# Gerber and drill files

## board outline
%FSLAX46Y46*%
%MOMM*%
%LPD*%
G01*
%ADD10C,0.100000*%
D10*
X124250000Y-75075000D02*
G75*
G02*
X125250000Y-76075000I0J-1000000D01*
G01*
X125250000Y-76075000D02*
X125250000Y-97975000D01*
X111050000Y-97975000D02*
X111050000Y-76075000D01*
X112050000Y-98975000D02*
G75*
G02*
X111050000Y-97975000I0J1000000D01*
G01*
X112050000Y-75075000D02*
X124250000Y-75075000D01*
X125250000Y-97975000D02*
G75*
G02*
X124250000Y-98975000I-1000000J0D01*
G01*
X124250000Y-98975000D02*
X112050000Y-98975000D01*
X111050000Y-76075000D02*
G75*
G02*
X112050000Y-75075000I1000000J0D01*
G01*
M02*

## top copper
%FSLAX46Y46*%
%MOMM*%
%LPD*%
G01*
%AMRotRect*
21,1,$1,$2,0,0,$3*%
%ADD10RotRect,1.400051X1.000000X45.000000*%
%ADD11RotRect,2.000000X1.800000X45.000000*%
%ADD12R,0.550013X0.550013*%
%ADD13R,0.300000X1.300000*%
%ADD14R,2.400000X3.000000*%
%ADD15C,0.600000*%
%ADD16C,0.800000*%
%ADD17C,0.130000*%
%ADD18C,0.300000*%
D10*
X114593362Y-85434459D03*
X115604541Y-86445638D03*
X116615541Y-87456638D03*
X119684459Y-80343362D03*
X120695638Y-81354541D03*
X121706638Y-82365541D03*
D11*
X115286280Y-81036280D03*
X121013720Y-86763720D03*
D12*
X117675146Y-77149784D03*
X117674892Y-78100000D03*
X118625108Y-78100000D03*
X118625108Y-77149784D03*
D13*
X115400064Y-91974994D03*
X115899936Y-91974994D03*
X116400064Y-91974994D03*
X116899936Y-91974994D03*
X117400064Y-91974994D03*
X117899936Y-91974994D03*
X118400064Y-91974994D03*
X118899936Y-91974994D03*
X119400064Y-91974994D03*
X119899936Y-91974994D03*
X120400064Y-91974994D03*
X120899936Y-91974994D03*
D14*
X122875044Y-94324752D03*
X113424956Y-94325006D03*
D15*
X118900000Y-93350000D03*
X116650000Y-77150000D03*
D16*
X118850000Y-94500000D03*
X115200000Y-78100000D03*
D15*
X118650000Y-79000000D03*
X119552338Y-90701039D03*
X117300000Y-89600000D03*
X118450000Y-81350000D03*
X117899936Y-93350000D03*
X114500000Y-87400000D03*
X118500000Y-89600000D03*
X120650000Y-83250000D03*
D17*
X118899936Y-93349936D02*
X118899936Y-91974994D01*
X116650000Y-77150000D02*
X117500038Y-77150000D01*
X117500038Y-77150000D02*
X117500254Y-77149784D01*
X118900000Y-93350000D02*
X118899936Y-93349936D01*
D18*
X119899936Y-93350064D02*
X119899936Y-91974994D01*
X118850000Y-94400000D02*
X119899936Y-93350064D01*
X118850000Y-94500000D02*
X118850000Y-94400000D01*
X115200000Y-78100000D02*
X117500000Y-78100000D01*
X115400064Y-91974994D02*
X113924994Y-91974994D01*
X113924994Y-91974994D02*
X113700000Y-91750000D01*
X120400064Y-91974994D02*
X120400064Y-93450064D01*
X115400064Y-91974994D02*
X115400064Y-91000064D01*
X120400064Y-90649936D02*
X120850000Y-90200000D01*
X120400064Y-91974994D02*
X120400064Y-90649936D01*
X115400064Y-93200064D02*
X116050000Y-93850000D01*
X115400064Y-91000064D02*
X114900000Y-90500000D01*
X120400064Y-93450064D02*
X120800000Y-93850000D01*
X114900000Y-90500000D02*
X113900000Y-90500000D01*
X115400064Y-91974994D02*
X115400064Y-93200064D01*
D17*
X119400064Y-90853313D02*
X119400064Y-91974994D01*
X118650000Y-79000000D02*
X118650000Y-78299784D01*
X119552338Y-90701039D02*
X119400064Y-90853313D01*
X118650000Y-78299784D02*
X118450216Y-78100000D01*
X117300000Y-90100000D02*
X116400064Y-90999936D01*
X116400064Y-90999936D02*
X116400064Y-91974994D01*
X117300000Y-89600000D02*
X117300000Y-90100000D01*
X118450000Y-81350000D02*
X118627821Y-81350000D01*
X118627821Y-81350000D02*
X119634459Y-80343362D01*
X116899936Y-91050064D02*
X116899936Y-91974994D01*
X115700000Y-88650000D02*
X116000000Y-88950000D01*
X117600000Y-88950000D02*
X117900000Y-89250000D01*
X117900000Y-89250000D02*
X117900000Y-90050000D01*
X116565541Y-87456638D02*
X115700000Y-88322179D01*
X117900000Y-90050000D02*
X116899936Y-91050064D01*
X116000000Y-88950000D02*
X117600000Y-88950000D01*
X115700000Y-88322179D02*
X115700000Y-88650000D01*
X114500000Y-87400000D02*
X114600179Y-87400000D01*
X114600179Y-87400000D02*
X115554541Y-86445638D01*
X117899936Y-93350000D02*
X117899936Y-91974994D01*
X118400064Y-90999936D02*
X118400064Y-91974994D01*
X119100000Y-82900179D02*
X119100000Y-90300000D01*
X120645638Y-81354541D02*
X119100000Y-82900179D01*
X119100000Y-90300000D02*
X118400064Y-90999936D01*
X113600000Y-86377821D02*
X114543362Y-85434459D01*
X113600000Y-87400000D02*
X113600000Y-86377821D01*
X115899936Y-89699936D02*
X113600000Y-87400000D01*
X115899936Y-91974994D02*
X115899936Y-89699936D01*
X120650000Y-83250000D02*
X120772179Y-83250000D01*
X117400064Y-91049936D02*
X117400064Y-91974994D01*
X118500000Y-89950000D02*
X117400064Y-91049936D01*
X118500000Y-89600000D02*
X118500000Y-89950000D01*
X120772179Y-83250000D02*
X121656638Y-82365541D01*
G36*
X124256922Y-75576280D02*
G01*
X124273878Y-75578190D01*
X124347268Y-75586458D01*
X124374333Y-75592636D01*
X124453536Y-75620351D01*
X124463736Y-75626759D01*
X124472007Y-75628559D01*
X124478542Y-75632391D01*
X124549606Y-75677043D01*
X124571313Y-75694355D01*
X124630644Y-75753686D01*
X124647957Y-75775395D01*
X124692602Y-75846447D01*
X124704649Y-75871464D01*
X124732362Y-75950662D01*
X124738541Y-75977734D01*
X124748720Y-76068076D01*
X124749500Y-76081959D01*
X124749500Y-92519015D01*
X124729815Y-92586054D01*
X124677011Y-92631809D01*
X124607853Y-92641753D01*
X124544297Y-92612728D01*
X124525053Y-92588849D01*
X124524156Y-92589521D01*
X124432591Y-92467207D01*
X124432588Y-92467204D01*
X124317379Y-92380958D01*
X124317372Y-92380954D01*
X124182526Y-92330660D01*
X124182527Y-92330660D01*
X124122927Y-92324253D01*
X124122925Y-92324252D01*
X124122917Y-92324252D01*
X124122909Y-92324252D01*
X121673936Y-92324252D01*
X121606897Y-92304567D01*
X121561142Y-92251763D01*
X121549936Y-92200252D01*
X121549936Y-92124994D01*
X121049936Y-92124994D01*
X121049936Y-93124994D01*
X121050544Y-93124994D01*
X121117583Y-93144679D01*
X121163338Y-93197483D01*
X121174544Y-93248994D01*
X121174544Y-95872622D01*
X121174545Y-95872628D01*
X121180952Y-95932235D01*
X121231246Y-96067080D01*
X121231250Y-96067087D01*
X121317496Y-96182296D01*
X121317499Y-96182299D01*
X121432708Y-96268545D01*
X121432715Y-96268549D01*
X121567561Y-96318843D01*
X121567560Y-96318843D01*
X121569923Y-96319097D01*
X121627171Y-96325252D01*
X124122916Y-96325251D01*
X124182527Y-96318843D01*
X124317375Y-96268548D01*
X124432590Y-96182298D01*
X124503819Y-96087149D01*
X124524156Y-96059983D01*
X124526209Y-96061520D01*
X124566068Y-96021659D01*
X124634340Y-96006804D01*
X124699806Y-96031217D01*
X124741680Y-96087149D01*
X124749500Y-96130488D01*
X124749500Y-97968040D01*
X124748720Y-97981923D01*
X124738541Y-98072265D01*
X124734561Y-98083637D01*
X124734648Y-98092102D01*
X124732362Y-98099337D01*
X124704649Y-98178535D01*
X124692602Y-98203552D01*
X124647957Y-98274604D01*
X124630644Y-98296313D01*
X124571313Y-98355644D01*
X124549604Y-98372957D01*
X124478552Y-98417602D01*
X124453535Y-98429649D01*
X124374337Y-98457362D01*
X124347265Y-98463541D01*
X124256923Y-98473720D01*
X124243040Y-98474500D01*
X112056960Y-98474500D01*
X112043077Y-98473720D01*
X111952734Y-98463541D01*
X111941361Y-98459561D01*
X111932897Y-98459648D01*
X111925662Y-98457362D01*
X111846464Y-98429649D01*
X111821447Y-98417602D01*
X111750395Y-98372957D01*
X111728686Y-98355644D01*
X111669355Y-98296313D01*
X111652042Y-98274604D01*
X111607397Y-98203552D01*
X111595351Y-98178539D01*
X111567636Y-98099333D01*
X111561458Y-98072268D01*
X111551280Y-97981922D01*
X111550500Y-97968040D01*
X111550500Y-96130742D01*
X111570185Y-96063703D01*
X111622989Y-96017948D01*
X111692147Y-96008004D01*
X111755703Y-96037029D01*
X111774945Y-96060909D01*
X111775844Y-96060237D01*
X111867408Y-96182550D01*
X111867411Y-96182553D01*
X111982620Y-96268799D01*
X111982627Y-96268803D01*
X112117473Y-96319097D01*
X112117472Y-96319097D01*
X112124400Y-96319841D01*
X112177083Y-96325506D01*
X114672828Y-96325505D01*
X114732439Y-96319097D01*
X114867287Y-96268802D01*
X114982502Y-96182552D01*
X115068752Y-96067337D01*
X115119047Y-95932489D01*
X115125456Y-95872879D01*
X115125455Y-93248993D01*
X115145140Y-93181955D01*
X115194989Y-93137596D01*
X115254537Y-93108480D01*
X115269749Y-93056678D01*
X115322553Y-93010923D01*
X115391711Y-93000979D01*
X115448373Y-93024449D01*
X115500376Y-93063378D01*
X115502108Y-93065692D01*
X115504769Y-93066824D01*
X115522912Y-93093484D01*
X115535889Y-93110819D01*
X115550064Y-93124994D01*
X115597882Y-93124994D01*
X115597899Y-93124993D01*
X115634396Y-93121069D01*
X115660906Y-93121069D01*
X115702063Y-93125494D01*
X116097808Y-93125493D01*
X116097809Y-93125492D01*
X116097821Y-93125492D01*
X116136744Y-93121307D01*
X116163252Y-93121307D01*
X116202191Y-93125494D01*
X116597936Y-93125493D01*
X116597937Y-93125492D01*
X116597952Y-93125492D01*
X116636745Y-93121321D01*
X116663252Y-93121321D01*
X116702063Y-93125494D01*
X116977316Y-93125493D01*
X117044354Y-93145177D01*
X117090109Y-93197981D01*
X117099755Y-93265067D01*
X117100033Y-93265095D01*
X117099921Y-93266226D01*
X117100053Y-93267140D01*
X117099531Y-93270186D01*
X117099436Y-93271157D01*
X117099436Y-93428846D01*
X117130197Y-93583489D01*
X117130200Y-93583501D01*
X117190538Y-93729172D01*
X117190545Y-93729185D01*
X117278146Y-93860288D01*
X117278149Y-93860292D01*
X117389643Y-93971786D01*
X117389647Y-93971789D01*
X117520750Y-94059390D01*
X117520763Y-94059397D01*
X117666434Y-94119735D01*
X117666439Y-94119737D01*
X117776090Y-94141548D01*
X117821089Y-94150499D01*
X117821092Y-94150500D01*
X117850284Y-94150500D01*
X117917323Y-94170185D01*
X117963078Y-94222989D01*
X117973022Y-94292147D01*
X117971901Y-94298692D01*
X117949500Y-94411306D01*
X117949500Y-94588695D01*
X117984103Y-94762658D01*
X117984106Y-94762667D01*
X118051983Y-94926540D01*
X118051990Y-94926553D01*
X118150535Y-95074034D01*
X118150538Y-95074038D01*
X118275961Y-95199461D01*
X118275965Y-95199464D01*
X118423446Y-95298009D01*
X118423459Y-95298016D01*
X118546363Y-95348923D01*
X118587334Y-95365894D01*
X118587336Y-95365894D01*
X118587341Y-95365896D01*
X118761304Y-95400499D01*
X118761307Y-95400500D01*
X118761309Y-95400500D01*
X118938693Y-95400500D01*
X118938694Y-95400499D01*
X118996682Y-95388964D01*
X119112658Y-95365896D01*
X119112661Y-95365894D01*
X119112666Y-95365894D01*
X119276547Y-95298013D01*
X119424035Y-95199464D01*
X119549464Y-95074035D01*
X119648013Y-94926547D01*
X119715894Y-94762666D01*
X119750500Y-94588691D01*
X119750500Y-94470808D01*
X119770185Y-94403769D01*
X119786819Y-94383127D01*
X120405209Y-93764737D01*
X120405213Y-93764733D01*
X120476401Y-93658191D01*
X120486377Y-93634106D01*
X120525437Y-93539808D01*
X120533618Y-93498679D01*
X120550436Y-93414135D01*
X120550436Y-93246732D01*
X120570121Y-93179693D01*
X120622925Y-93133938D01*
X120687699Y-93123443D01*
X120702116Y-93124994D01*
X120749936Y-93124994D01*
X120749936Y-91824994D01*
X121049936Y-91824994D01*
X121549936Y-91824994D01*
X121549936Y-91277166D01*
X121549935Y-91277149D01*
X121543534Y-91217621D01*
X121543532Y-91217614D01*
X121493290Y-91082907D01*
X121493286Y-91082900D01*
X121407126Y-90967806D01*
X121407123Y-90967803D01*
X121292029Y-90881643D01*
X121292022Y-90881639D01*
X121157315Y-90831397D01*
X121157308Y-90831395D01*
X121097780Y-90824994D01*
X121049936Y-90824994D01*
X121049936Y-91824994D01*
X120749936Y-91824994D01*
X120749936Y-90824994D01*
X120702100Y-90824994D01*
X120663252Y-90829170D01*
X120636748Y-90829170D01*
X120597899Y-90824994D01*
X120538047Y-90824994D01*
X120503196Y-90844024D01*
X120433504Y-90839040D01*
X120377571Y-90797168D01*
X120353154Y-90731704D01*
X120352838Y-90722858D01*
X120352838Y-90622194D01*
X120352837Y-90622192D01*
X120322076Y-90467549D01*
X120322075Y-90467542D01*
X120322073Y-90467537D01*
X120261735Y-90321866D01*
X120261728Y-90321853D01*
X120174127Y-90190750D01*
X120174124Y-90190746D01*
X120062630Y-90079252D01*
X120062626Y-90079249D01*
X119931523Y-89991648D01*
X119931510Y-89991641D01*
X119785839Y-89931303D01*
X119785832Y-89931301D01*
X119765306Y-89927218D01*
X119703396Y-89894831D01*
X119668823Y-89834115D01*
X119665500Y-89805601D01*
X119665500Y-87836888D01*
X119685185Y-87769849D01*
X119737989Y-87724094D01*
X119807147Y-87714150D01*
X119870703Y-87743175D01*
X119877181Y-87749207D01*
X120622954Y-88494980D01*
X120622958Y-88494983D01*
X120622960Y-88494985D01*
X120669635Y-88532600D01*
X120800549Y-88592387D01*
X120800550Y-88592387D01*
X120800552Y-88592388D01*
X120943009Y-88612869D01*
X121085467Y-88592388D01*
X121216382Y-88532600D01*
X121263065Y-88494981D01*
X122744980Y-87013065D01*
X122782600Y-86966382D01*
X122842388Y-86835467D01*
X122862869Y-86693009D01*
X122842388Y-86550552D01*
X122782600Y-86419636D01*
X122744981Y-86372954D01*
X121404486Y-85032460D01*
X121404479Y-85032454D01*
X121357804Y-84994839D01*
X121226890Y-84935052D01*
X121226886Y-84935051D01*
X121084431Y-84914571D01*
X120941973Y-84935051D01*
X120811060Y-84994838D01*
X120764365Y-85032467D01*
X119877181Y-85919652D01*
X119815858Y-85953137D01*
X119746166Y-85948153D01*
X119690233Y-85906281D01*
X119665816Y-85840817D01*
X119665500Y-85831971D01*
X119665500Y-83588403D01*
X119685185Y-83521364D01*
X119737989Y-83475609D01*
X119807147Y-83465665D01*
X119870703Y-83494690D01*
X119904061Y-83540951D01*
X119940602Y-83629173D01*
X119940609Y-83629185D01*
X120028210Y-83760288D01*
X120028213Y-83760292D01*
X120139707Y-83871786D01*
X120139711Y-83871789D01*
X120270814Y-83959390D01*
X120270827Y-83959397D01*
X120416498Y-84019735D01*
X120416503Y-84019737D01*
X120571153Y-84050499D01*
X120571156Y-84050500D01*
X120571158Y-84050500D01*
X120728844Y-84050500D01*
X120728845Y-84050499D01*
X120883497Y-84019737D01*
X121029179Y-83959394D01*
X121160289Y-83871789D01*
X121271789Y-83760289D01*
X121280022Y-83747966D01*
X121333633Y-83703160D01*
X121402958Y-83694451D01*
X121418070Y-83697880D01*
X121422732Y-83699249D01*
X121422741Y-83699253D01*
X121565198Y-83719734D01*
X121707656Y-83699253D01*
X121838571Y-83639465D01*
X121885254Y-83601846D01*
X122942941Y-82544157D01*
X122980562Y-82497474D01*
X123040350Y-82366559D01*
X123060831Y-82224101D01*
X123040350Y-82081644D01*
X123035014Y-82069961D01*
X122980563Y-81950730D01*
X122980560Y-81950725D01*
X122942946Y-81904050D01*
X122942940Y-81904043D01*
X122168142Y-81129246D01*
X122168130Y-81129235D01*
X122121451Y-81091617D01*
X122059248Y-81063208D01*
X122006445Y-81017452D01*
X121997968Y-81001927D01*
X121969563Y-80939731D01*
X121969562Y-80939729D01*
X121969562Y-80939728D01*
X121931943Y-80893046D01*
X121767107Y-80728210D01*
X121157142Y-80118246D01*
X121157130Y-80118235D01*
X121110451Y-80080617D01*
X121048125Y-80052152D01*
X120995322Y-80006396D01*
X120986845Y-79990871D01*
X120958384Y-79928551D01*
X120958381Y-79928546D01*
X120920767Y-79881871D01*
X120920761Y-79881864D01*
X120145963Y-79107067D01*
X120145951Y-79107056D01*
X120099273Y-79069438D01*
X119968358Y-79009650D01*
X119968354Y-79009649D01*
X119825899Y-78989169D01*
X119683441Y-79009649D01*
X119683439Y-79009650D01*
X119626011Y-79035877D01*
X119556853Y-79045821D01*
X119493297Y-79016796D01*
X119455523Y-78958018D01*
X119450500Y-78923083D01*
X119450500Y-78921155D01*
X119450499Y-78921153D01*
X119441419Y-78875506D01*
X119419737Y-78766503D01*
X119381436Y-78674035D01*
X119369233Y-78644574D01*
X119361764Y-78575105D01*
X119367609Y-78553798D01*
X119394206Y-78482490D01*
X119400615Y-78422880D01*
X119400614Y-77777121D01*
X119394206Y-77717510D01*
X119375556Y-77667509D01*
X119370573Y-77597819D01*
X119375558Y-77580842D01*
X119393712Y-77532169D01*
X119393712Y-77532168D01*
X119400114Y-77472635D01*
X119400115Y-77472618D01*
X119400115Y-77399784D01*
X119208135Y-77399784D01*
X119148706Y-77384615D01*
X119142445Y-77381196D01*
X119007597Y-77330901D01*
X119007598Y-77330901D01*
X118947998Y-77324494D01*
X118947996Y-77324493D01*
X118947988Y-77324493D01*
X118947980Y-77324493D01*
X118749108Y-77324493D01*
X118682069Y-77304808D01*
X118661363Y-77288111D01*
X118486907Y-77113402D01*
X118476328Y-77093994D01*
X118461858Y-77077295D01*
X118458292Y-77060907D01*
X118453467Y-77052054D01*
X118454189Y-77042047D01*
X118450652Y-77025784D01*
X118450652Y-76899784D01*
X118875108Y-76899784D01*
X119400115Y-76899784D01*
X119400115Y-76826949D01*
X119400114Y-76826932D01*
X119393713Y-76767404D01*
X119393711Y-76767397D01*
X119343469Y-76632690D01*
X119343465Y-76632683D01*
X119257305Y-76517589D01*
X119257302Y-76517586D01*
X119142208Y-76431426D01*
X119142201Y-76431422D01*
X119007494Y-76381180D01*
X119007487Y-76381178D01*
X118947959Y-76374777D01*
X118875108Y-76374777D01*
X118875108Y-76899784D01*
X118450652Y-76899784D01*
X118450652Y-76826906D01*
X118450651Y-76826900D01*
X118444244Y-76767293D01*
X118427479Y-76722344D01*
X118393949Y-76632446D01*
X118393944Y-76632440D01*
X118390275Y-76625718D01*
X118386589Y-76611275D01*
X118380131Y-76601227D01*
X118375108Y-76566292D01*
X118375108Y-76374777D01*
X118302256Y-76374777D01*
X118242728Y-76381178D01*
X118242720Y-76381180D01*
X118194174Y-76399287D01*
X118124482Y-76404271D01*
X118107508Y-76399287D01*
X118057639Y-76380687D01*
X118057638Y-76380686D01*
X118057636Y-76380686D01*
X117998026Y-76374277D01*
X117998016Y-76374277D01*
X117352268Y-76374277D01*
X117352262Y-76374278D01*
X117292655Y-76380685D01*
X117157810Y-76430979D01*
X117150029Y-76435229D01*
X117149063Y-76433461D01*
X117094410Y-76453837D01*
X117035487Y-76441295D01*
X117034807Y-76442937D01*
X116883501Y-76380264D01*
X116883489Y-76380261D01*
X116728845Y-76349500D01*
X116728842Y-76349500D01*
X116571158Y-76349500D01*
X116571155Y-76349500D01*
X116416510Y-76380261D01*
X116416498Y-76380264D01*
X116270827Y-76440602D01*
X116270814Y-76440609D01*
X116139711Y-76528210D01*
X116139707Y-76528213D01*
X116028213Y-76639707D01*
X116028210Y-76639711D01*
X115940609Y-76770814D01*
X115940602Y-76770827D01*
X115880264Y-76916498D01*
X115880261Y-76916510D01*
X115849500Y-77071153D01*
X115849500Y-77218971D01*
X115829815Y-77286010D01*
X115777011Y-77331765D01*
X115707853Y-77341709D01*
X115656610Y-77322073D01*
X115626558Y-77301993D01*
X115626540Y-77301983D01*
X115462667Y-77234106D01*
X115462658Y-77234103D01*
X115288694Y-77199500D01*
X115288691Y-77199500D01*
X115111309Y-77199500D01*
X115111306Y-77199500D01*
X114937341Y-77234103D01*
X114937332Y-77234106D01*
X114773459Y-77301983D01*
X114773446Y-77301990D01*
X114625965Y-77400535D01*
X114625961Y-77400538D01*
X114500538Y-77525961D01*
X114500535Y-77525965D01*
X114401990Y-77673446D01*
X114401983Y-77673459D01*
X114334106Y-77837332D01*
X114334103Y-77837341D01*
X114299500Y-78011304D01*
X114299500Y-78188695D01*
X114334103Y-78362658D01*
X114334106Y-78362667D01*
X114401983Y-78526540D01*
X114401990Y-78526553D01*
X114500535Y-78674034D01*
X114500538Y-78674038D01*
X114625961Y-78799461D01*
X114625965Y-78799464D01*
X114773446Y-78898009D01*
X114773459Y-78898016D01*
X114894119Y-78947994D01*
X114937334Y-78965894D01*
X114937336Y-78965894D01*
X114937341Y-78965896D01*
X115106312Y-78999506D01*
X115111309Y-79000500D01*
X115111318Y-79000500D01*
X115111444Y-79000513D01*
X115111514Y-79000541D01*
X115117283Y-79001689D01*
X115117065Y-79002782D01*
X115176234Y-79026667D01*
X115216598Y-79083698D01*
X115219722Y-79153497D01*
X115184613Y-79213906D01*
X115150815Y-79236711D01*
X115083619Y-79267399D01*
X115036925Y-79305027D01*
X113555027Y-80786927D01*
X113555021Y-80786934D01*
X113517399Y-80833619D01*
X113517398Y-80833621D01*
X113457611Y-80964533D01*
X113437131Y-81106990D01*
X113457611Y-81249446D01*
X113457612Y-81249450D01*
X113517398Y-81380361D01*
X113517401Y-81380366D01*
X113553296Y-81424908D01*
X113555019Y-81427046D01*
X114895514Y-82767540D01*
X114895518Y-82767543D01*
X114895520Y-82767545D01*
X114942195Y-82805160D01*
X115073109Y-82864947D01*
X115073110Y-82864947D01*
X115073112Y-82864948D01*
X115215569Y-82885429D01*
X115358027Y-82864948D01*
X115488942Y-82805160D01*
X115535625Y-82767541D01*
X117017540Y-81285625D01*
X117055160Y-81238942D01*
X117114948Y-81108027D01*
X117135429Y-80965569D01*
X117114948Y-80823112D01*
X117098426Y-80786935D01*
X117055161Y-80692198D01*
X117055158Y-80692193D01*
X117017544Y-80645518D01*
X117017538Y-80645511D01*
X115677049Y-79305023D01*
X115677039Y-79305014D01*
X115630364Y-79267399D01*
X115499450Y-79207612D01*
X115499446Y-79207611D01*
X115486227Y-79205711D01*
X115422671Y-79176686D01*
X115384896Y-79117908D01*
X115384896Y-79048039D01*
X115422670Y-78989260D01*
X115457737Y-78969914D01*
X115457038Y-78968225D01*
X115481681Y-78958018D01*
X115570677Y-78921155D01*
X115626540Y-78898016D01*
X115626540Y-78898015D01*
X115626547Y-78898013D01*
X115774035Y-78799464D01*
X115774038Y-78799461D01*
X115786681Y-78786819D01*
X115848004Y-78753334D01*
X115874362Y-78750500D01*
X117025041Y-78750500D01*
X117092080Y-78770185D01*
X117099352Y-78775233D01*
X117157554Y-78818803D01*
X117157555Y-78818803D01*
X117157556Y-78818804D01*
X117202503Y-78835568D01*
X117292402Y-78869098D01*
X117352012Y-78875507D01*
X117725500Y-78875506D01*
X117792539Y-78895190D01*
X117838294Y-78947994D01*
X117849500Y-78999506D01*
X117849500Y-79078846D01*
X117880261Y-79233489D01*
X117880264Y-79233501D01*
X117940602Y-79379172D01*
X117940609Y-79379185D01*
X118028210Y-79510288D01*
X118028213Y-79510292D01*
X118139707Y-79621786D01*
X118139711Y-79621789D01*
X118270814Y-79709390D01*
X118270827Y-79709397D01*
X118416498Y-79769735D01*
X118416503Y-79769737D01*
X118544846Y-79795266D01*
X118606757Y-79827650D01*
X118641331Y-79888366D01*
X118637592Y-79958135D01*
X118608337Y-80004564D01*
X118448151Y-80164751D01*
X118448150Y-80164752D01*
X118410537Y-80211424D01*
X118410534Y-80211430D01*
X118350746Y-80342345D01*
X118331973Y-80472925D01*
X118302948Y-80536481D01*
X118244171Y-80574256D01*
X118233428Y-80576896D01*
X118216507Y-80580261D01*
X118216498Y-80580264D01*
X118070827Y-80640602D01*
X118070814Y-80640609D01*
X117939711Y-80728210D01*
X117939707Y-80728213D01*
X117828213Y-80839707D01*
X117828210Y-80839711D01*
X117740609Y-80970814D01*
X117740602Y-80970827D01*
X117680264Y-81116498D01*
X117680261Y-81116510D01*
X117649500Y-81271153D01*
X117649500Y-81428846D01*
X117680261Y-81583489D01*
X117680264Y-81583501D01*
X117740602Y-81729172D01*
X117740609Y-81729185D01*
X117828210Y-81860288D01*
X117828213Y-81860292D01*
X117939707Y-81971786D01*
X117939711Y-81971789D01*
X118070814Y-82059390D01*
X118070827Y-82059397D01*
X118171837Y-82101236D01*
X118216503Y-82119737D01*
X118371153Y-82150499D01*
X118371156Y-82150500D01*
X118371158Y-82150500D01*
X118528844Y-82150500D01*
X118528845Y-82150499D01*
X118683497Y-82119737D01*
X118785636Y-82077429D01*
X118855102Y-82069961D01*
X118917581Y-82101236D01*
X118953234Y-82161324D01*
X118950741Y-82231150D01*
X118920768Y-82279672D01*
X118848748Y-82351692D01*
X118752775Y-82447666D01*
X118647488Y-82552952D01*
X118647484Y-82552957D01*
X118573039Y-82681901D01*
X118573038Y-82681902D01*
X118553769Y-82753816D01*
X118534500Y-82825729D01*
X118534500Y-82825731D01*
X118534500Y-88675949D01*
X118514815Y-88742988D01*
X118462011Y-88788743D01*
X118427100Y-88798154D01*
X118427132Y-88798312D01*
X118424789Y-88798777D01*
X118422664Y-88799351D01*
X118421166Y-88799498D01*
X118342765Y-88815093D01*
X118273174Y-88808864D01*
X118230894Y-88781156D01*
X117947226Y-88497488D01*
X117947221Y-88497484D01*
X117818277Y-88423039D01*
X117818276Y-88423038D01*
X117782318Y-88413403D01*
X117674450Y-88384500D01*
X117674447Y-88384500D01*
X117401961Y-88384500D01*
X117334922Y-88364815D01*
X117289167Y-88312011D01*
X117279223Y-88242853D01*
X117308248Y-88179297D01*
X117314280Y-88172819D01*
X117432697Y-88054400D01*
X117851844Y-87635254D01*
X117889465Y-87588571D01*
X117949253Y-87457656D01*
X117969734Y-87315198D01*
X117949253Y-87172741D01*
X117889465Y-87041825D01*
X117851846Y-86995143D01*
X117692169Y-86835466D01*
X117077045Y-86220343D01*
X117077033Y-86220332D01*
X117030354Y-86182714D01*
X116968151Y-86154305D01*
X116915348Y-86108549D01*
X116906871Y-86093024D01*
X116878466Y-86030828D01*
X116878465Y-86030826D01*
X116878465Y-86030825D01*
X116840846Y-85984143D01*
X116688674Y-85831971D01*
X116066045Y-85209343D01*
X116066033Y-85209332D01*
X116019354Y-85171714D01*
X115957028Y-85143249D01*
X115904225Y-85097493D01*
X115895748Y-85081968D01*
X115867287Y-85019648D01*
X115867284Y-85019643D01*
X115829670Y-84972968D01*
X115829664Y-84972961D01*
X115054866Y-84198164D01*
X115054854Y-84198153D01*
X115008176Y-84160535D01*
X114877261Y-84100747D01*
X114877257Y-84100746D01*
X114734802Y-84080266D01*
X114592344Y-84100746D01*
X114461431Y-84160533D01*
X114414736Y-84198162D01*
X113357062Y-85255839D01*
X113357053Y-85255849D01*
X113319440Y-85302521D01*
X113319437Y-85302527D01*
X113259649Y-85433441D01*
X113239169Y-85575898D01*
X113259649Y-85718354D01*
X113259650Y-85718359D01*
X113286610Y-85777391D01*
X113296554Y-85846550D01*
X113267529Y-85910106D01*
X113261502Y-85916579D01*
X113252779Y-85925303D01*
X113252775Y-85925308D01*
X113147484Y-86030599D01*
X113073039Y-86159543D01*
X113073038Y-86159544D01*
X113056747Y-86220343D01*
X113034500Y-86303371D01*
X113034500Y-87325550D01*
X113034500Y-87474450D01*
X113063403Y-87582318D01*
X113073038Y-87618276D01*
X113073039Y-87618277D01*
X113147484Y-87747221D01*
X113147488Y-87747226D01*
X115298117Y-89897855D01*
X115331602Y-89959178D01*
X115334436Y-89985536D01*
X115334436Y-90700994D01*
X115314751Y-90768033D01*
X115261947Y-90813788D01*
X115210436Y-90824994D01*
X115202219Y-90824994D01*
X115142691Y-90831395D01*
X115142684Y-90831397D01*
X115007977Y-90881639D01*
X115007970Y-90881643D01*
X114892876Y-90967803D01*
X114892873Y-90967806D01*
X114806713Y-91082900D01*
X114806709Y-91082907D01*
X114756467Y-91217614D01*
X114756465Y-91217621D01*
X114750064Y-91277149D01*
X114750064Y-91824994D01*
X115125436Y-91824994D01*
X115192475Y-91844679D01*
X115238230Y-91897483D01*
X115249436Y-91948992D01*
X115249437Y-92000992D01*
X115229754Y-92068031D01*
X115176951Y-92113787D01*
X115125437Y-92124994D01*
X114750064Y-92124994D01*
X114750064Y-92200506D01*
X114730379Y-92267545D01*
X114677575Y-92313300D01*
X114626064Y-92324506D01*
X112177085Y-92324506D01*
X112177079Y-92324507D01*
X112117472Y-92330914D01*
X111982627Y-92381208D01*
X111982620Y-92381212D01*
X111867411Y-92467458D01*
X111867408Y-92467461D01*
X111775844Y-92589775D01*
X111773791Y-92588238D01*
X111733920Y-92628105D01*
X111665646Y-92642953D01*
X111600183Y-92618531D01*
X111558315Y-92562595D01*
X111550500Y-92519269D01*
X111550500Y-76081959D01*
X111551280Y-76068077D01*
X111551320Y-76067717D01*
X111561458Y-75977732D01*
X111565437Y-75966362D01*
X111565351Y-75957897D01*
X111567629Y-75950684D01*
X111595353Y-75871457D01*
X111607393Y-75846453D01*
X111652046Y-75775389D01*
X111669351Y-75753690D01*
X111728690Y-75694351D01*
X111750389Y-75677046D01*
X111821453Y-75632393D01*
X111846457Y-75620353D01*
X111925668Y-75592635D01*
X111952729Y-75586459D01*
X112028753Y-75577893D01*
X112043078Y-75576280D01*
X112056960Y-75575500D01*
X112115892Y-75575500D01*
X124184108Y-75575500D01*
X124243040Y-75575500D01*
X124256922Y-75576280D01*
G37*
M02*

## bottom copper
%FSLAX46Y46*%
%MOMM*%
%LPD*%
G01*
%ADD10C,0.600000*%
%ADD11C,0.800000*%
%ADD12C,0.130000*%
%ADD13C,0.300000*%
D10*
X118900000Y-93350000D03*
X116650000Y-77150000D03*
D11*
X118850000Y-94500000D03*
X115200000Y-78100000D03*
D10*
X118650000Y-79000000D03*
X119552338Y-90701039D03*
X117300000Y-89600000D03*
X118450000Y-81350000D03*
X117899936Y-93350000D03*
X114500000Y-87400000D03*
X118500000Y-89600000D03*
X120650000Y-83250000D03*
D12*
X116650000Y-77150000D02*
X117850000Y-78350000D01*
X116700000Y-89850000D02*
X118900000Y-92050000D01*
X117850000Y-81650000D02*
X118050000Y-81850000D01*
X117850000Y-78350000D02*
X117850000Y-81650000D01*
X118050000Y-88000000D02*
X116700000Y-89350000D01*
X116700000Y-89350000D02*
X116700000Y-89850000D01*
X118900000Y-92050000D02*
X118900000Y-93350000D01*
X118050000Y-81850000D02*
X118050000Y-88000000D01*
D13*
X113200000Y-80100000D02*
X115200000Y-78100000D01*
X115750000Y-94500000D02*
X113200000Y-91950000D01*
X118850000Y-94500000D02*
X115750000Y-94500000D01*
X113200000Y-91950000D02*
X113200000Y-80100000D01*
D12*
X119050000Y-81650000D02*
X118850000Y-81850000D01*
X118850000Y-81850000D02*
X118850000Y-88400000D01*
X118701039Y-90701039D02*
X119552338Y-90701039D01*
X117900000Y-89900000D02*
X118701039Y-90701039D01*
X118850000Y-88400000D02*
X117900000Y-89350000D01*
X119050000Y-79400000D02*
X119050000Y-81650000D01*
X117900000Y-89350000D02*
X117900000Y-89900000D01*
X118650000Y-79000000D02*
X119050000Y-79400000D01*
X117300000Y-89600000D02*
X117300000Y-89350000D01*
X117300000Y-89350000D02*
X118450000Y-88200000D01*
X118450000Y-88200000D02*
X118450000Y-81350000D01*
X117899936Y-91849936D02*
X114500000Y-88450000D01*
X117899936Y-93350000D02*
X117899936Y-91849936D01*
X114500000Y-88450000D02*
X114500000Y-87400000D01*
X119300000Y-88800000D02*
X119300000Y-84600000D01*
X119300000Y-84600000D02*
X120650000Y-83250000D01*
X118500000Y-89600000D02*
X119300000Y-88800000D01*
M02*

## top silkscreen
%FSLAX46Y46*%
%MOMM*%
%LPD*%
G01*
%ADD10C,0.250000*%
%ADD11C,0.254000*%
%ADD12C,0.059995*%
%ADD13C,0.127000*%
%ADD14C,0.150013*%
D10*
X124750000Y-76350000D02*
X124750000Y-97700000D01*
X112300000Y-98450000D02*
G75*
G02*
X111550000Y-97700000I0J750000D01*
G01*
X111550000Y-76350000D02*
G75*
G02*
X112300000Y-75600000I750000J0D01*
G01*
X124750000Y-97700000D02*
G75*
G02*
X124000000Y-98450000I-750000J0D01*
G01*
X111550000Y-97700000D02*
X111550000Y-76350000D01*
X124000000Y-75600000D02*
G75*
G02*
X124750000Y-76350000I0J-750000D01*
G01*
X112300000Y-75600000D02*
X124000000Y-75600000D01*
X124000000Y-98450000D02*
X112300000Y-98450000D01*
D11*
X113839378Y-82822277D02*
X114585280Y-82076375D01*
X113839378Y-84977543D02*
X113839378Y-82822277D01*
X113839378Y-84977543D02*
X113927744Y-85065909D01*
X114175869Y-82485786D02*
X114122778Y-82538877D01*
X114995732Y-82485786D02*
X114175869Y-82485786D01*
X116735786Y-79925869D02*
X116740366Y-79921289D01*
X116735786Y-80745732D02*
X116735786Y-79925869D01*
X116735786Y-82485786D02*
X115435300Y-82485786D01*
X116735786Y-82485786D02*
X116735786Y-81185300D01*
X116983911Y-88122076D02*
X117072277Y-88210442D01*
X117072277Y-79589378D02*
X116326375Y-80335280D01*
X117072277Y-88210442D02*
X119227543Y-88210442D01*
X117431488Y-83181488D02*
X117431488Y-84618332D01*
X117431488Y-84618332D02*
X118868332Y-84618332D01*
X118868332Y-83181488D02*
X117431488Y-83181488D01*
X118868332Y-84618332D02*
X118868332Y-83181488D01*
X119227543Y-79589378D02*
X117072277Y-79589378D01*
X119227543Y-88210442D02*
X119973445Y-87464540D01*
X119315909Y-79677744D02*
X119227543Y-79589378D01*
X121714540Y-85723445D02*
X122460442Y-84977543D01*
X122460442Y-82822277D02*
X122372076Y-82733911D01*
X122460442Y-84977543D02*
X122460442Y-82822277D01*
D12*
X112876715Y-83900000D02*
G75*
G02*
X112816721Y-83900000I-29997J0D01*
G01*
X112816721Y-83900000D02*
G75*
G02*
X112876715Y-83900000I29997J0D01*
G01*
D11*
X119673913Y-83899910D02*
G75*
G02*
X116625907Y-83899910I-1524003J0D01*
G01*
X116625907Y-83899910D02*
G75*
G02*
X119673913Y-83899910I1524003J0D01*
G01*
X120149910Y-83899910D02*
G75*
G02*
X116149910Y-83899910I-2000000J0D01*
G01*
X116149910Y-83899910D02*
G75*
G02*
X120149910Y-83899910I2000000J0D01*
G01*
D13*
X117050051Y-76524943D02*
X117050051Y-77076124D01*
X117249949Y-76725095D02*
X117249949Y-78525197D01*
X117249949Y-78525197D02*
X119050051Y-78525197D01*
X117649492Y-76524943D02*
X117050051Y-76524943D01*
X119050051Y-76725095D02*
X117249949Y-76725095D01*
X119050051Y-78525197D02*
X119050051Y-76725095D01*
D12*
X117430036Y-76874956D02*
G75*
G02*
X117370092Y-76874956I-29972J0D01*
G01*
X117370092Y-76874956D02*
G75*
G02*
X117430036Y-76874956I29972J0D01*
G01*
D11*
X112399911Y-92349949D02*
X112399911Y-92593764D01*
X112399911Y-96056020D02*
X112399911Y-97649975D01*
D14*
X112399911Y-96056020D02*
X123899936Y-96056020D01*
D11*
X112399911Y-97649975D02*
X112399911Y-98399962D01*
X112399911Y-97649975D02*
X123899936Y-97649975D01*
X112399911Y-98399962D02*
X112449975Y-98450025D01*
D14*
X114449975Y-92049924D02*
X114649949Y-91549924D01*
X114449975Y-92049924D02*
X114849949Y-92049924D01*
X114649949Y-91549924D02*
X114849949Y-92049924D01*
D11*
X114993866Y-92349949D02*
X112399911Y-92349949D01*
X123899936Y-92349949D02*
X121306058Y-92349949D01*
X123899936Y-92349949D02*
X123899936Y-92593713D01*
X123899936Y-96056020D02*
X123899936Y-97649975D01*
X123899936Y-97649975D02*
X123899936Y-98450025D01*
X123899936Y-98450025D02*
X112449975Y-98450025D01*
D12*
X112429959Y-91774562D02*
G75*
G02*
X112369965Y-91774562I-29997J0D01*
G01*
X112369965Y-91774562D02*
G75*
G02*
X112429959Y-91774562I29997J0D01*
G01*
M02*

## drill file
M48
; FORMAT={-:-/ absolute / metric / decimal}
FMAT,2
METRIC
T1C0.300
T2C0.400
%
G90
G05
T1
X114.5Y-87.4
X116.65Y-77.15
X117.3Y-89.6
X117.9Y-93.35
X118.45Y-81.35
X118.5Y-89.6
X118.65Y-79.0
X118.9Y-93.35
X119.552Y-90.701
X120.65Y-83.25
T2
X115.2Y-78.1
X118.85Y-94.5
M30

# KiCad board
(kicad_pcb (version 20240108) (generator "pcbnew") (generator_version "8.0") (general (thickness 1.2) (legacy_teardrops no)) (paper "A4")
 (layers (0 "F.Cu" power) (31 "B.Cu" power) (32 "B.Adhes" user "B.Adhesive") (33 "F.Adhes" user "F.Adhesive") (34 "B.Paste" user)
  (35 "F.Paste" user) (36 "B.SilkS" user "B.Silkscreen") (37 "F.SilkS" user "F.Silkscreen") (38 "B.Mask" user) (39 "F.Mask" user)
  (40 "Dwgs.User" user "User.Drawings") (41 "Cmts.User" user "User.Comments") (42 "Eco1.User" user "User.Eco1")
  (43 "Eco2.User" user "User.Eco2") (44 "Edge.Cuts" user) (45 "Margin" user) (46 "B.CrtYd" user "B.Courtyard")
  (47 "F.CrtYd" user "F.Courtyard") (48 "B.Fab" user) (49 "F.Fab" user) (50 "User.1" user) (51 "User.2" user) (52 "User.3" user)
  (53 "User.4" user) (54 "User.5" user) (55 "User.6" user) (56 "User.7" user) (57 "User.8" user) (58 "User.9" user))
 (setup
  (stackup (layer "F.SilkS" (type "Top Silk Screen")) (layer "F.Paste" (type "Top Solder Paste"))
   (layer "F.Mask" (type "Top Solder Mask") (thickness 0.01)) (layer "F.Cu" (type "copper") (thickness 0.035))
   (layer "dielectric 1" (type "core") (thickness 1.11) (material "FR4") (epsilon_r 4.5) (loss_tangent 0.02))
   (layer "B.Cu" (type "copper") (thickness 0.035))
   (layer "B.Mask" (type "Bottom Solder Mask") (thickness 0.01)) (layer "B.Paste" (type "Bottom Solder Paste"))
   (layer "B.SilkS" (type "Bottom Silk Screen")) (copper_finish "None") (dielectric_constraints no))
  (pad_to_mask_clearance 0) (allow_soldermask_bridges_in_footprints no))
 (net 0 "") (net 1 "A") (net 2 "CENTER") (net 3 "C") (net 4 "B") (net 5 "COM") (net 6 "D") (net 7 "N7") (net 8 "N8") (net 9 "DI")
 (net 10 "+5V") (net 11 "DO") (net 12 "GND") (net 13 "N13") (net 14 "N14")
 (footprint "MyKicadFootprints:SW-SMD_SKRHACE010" (layer "F.Cu") (at 118.15 83.9 45)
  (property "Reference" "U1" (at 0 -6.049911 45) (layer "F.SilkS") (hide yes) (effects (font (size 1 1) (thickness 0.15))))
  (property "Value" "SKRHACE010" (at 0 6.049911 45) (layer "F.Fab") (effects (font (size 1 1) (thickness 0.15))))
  (fp_line (start -2.286005 -3.810135) (end -1.23114 -3.810135) (stroke (width 0.254) (type solid)) (layer "F.SilkS"))
  (fp_line (start -3.810008 -2.286132) (end -2.286005 -3.810135) (stroke (width 0.254) (type solid)) (layer "F.SilkS"))
  (fp_line (start -3.810008 -2.286132) (end -3.810008 -2.161164) (stroke (width 0.254) (type solid)) (layer "F.SilkS"))
  (fp_line (start -1.810135 -3.810135) (end -1.885217 -3.810135) (stroke (width 0.254) (type solid)) (layer "F.SilkS"))
  (fp_line (start -1.230404 -3.230405) (end -1.810135 -3.810135) (stroke (width 0.254) (type solid)) (layer "F.SilkS"))
  (fp_line (start 1.810135 -3.810135) (end 1.816612 -3.810135) (stroke (width 0.254) (type solid)) (layer "F.SilkS"))
  (fp_line (start 1.230404 -3.230405) (end 1.810135 -3.810135) (stroke (width 0.254) (type solid)) (layer "F.SilkS"))
  (fp_line (start 0 -2.000001) (end -0.919582 -2.919583) (stroke (width 0.254) (type solid)) (layer "F.SilkS"))
  (fp_line (start 0 -2.000001) (end 0.919582 -2.919583) (stroke (width 0.254) (type solid)) (layer "F.SilkS"))
  (fp_line (start -3.810008 2.160909) (end -3.810008 2.285878) (stroke (width 0.254) (type solid)) (layer "F.SilkS"))
  (fp_line (start 2.286005 -3.810135) (end 1.23114 -3.810135) (stroke (width 0.254) (type solid)) (layer "F.SilkS"))
  (fp_line (start -3.810008 2.285878) (end -2.286005 3.809881) (stroke (width 0.254) (type solid)) (layer "F.SilkS"))
  (fp_line (start 0 -1.016129) (end -1.016002 -0.000127) (stroke (width 0.254) (type solid)) (layer "F.SilkS"))
  (fp_line (start -1.016002 -0.000127) (end 0 1.015875) (stroke (width 0.254) (type solid)) (layer "F.SilkS"))
  (fp_line (start 1.016002 -0.000127) (end 0 -1.016129) (stroke (width 0.254) (type solid)) (layer "F.SilkS"))
  (fp_line (start 0 1.015875) (end 1.016002 -0.000127) (stroke (width 0.254) (type solid)) (layer "F.SilkS"))
  (fp_line (start 3.810008 -2.286132) (end 2.286005 -3.810135) (stroke (width 0.254) (type solid)) (layer "F.SilkS"))
  (fp_line (start -2.286005 3.809881) (end -1.23114 3.809881) (stroke (width 0.254) (type solid)) (layer "F.SilkS"))
  (fp_line (start 3.810008 -2.161164) (end 3.810008 -2.286132) (stroke (width 0.254) (type solid)) (layer "F.SilkS"))
  (fp_line (start 1.23114 3.809881) (end 2.286005 3.809881) (stroke (width 0.254) (type solid)) (layer "F.SilkS"))
  (fp_line (start 3.810008 2.285878) (end 3.810008 2.160909) (stroke (width 0.254) (type solid)) (layer "F.SilkS"))
  (fp_line (start 2.286005 3.809881) (end 3.810008 2.285878) (stroke (width 0.254) (type solid)) (layer "F.SilkS"))
  (fp_circle (center -3.749987 -3.749987) (end -3.71999 -3.749987) (stroke (width 0.059995) (type solid)) (fill none) (layer "F.SilkS"))
  (fp_circle (center 0 -0.000127) (end 1.524003 -0.000127) (stroke (width 0.254) (type solid)) (fill none) (layer "F.SilkS"))
  (fp_circle (center 0 -0.000127) (end 2 -0.000127) (stroke (width 0.254) (type solid)) (fill none) (layer "F.SilkS"))
  (pad "1" smd rect (at -3.599949 -1.429896 45) (size 1.400051 1) (layers "F.Cu" "F.Paste" "F.Mask") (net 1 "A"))
  (pad "2" smd rect (at -3.599949 0.000127 45) (size 1.400051 1) (layers "F.Cu" "F.Paste" "F.Mask") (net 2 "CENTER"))
  (pad "3" smd rect (at -3.599949 1.429896 45) (size 1.400051 1) (layers "F.Cu" "F.Paste" "F.Mask") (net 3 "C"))
  (pad "4" smd rect (at 3.599949 -1.429896 45) (size 1.400051 1) (layers "F.Cu" "F.Paste" "F.Mask") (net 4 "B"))
  (pad "5" smd rect (at 3.599949 0.000127 45) (size 1.400051 1) (layers "F.Cu" "F.Paste" "F.Mask") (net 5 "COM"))
  (pad "6" smd rect (at 3.599949 1.429896 45) (size 1.400051 1) (layers "F.Cu" "F.Paste" "F.Mask") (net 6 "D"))
  (pad "7" smd rect (at 0 -4.049912 45) (size 2 1.8) (layers "F.Cu" "F.Paste" "F.Mask") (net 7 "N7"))
  (pad "8" smd rect (at 0 4.049912 45) (size 2 1.8) (layers "F.Cu" "F.Paste" "F.Mask") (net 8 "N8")))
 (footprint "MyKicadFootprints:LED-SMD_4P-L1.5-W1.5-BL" (layer "F.Cu") (at 118.15 77.624892 -90)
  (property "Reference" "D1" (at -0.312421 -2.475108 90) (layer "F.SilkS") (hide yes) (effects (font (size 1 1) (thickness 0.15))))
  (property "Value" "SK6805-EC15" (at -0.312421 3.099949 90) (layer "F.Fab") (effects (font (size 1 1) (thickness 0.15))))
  (fp_line (start -1.099949 1.099949) (end -0.548768 1.099949) (stroke (width 0.127) (type solid)) (layer "F.SilkS"))
  (fp_line (start -0.899797 0.900051) (end 0.900305 0.900051) (stroke (width 0.127) (type solid)) (layer "F.SilkS"))
  (fp_line (start 0.900305 0.900051) (end 0.900305 -0.900051) (stroke (width 0.127) (type solid)) (layer "F.SilkS"))
  (fp_line (start -1.099949 0.500508) (end -1.099949 1.099949) (stroke (width 0.127) (type solid)) (layer "F.SilkS"))
  (fp_line (start -0.899797 -0.900051) (end -0.899797 0.900051) (stroke (width 0.127) (type solid)) (layer "F.SilkS"))
  (fp_line (start 0.900305 -0.900051) (end -0.899797 -0.900051) (stroke (width 0.127) (type solid)) (layer "F.SilkS"))
  (fp_circle (center -0.749936 0.749936) (end -0.719964 0.749936) (stroke (width 0.059995) (type solid)) (fill none) (layer "F.SilkS"))
  (pad "1" smd rect (at -0.475108 0.474854 270) (size 0.550013 0.550013) (layers "F.Cu" "F.Paste" "F.Mask") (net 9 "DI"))
  (pad "2" smd rect (at 0.475108 0.475108 270) (size 0.550013 0.550013) (layers "F.Cu" "F.Paste" "F.Mask") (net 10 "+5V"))
  (pad "3" smd rect (at 0.475108 -0.475108 270) (size 0.550013 0.550013) (layers "F.Cu" "F.Paste" "F.Mask") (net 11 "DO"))
  (pad "4" smd rect (at -0.475108 -0.475108 270) (size 0.550013 0.550013) (layers "F.Cu" "F.Paste" "F.Mask") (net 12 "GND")))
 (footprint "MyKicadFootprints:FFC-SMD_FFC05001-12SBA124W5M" (layer "F.Cu") (at 118.15 93.15)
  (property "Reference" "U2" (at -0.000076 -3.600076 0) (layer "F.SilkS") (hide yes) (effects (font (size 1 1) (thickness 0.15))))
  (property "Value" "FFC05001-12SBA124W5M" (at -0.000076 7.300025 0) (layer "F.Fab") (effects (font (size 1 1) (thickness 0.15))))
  (fp_line (start -5.750089 -0.800051) (end -5.750089 -0.556236) (stroke (width 0.254) (type solid)) (layer "F.SilkS"))
  (fp_line (start -5.750089 2.90602) (end -5.750089 4.499975) (stroke (width 0.254) (type solid)) (layer "F.SilkS"))
  (fp_line (start -5.750089 2.90602) (end 5.749936 2.90602) (stroke (width 0.150013) (type solid)) (layer "F.SilkS"))
  (fp_line (start -5.750089 4.499975) (end -5.750089 5.249962) (stroke (width 0.254) (type solid)) (layer "F.SilkS"))
  (fp_line (start -5.750089 4.499975) (end 5.749936 4.499975) (stroke (width 0.254) (type solid)) (layer "F.SilkS"))
  (fp_line (start -5.750089 5.249962) (end -5.700025 5.300025) (stroke (width 0.254) (type solid)) (layer "F.SilkS"))
  (fp_line (start -3.700025 -1.100076) (end -3.500051 -1.600076) (stroke (width 0.150013) (type solid)) (layer "F.SilkS"))
  (fp_line (start -3.700025 -1.100076) (end -3.300051 -1.100076) (stroke (width 0.150013) (type solid)) (layer "F.SilkS"))
  (fp_line (start -3.500051 -1.600076) (end -3.300051 -1.100076) (stroke (width 0.150013) (type solid)) (layer "F.SilkS"))
  (fp_line (start -3.156134 -0.800051) (end -5.750089 -0.800051) (stroke (width 0.254) (type solid)) (layer "F.SilkS"))
  (fp_line (start 5.749936 -0.800051) (end 3.156058 -0.800051) (stroke (width 0.254) (type solid)) (layer "F.SilkS"))
  (fp_line (start 5.749936 -0.800051) (end 5.749936 -0.556287) (stroke (width 0.254) (type solid)) (layer "F.SilkS"))
  (fp_line (start 5.749936 2.90602) (end 5.749936 4.499975) (stroke (width 0.254) (type solid)) (layer "F.SilkS"))
  (fp_line (start 5.749936 4.499975) (end 5.749936 5.300025) (stroke (width 0.254) (type solid)) (layer "F.SilkS"))
  (fp_line (start 5.749936 5.300025) (end -5.700025 5.300025) (stroke (width 0.254) (type solid)) (layer "F.SilkS"))
  (fp_circle (center -5.750038 -1.375438) (end -5.720041 -1.375438) (stroke (width 0.059995) (type solid)) (fill none) (layer "F.SilkS"))
  (pad "1" smd rect (at -2.749936 -1.175006) (size 0.3 1.3) (layers "F.Cu" "F.Paste" "F.Mask") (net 12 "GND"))
  (pad "2" smd rect (at -2.250064 -1.175006) (size 0.3 1.3) (layers "F.Cu" "F.Paste" "F.Mask") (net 1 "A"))
  (pad "3" smd rect (at -1.749936 -1.175006) (size 0.3 1.3) (layers "F.Cu" "F.Paste" "F.Mask") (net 4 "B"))
  (pad "4" smd rect (at -1.250064 -1.175006) (size 0.3 1.3) (layers "F.Cu" "F.Paste" "F.Mask") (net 3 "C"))
  (pad "5" smd rect (at -0.749936 -1.175006) (size 0.3 1.3) (layers "F.Cu" "F.Paste" "F.Mask") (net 6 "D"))
  (pad "6" smd rect (at -0.250064 -1.175006) (size 0.3 1.3) (layers "F.Cu" "F.Paste" "F.Mask") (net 2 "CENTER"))
  (pad "7" smd rect (at 0.250064 -1.175006) (size 0.3 1.3) (layers "F.Cu" "F.Paste" "F.Mask") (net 5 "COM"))
  (pad "8" smd rect (at 0.749936 -1.175006) (size 0.3 1.3) (layers "F.Cu" "F.Paste" "F.Mask") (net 9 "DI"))
  (pad "9" smd rect (at 1.250064 -1.175006) (size 0.3 1.3) (layers "F.Cu" "F.Paste" "F.Mask") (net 11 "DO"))
  (pad "10" smd rect (at 1.749936 -1.175006) (size 0.3 1.3) (layers "F.Cu" "F.Paste" "F.Mask") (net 10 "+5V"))
  (pad "11" smd rect (at 2.250064 -1.175006) (size 0.3 1.3) (layers "F.Cu" "F.Paste" "F.Mask") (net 12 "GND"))
  (pad "12" smd rect (at 2.749936 -1.175006) (size 0.3 1.3) (layers "F.Cu" "F.Paste" "F.Mask") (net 12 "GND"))
  (pad "13" smd rect (at 4.725044 1.174752) (size 2.4 3) (layers "F.Cu" "F.Paste" "F.Mask") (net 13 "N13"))
  (pad "14" smd rect (at -4.725044 1.175006) (size 2.4 3) (layers "F.Cu" "F.Paste" "F.Mask") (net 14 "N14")))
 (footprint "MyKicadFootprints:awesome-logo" (layer "B.Cu") (at 121.45 78.95 -90)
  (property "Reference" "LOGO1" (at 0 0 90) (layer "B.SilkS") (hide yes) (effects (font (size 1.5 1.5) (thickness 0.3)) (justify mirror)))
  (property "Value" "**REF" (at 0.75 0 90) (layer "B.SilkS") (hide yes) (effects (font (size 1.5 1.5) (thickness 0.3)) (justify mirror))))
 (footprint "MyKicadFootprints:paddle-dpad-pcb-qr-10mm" (layer "B.Cu") (at 119.35 87.3 180)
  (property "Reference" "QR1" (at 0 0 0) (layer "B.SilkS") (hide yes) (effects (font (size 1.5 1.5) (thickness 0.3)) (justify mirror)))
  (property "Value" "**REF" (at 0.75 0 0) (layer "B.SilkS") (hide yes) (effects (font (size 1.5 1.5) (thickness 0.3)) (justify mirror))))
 (gr_line (start 124.75 76.35) (end 124.75 97.7) (stroke (width 0.25) (type default)) (layer "F.SilkS"))
 (gr_arc (start 112.3 98.45) (mid 111.76967 98.23033) (end 111.55 97.7) (stroke (width 0.25) (type default)) (layer "F.SilkS"))
 (gr_arc (start 111.55 76.35) (mid 111.76967 75.81967) (end 112.3 75.6) (stroke (width 0.25) (type default)) (layer "F.SilkS"))
 (gr_arc (start 124.75 97.7) (mid 124.53033 98.23033) (end 124 98.45) (stroke (width 0.25) (type default)) (layer "F.SilkS"))
 (gr_line (start 111.55 97.7) (end 111.55 76.35) (stroke (width 0.25) (type default)) (layer "F.SilkS"))
 (gr_arc (start 124 75.6) (mid 124.53033 75.81967) (end 124.75 76.35) (stroke (width 0.25) (type default)) (layer "F.SilkS"))
 (gr_line (start 112.3 75.6) (end 124 75.6) (stroke (width 0.25) (type default)) (layer "F.SilkS"))
 (gr_line (start 124 98.45) (end 112.3 98.45) (stroke (width 0.25) (type default)) (layer "F.SilkS"))
 (gr_arc (start 124.25 75.075) (mid 124.957107 75.367893) (end 125.25 76.075) (stroke (width 0.1) (type default)) (layer "Edge.Cuts"))
 (gr_line (start 125.25 76.075) (end 125.25 97.975) (stroke (width 0.1) (type default)) (layer "Edge.Cuts"))
 (gr_line (start 111.05 97.975) (end 111.05 76.075) (stroke (width 0.1) (type default)) (layer "Edge.Cuts"))
 (gr_arc (start 112.05 98.975) (mid 111.342893 98.682107) (end 111.05 97.975) (stroke (width 0.1) (type default)) (layer "Edge.Cuts"))
 (gr_line (start 112.05 75.075) (end 124.25 75.075) (stroke (width 0.1) (type default)) (layer "Edge.Cuts"))
 (gr_arc (start 125.25 97.975) (mid 124.957107 98.682107) (end 124.25 98.975) (stroke (width 0.1) (type default)) (layer "Edge.Cuts"))
 (gr_line (start 124.25 98.975) (end 112.05 98.975) (stroke (width 0.1) (type default)) (layer "Edge.Cuts"))
 (gr_arc (start 111.05 76.075) (mid 111.342893 75.367893) (end 112.05 75.075) (stroke (width 0.1) (type default)) (layer "Edge.Cuts"))
 (segment (start 118.899936 93.349936) (end 118.899936 91.974994) (width 0.13) (layer "F.Cu") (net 9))
 (segment (start 116.65 77.15) (end 117.500038 77.15) (width 0.13) (layer "F.Cu") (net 9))
 (segment (start 117.500038 77.15) (end 117.500254 77.149784) (width 0.13) (layer "F.Cu") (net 9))
 (segment (start 118.9 93.35) (end 118.899936 93.349936) (width 0.13) (layer "F.Cu") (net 9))
 (via (at 118.9 93.35) (size 0.6) (drill 0.3) (layers "F.Cu" "B.Cu") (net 9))
 (via (at 116.65 77.15) (size 0.6) (drill 0.3) (layers "F.Cu" "B.Cu") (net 9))
 (segment (start 116.65 77.15) (end 117.85 78.35) (width 0.13) (layer "B.Cu") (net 9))
 (segment (start 116.7 89.85) (end 118.9 92.05) (width 0.13) (layer "B.Cu") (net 9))
 (segment (start 117.85 81.65) (end 118.05 81.85) (width 0.13) (layer "B.Cu") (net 9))
 (segment (start 117.85 78.35) (end 117.85 81.65) (width 0.13) (layer "B.Cu") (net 9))
 (segment (start 118.05 88) (end 116.7 89.35) (width 0.13) (layer "B.Cu") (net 9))
 (segment (start 116.7 89.35) (end 116.7 89.85) (width 0.13) (layer "B.Cu") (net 9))
 (segment (start 118.9 92.05) (end 118.9 93.35) (width 0.13) (layer "B.Cu") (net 9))
 (segment (start 118.05 81.85) (end 118.05 88) (width 0.13) (layer "B.Cu") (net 9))
 (segment (start 119.899936 93.350064) (end 119.899936 91.974994) (width 0.3) (layer "F.Cu") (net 10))
 (segment (start 118.85 94.4) (end 119.899936 93.350064) (width 0.3) (layer "F.Cu") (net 10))
 (segment (start 118.85 94.5) (end 118.85 94.4) (width 0.3) (layer "F.Cu") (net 10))
 (segment (start 115.2 78.1) (end 117.5 78.1) (width 0.3) (layer "F.Cu") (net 10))
 (via (at 118.85 94.5) (size 0.8) (drill 0.4) (layers "F.Cu" "B.Cu") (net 10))
 (via (at 115.2 78.1) (size 0.8) (drill 0.4) (layers "F.Cu" "B.Cu") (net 10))
 (segment (start 113.2 80.1) (end 115.2 78.1) (width 0.3) (layer "B.Cu") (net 10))
 (segment (start 115.75 94.5) (end 113.2 91.95) (width 0.3) (layer "B.Cu") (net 10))
 (segment (start 118.85 94.5) (end 115.75 94.5) (width 0.3) (layer "B.Cu") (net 10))
 (segment (start 113.2 91.95) (end 113.2 80.1) (width 0.3) (layer "B.Cu") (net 10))
 (segment (start 115.400064 91.974994) (end 113.924994 91.974994) (width 0.3) (layer "F.Cu") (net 12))
 (segment (start 113.924994 91.974994) (end 113.7 91.75) (width 0.3) (layer "F.Cu") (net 12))
 (segment (start 120.400064 91.974994) (end 120.400064 93.450064) (width 0.3) (layer "F.Cu") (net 12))
 (segment (start 115.400064 91.974994) (end 115.400064 91.000064) (width 0.3) (layer "F.Cu") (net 12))
 (segment (start 120.400064 90.649936) (end 120.85 90.2) (width 0.3) (layer "F.Cu") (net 12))
 (segment (start 120.400064 91.974994) (end 120.400064 90.649936) (width 0.3) (layer "F.Cu") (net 12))
 (segment (start 115.400064 93.200064) (end 116.05 93.85) (width 0.3) (layer "F.Cu") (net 12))
 (segment (start 115.400064 91.000064) (end 114.9 90.5) (width 0.3) (layer "F.Cu") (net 12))
 (segment (start 120.400064 93.450064) (end 120.8 93.85) (width 0.3) (layer "F.Cu") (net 12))
 (segment (start 114.9 90.5) (end 113.9 90.5) (width 0.3) (layer "F.Cu") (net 12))
 (segment (start 115.400064 91.974994) (end 115.400064 93.200064) (width 0.3) (layer "F.Cu") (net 12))
 (segment (start 119.400064 90.853313) (end 119.400064 91.974994) (width 0.13) (layer "F.Cu") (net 11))
 (segment (start 118.65 79) (end 118.65 78.299784) (width 0.13) (layer "F.Cu") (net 11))
 (segment (start 119.552338 90.701039) (end 119.400064 90.853313) (width 0.13) (layer "F.Cu") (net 11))
 (segment (start 118.65 78.299784) (end 118.450216 78.1) (width 0.13) (layer "F.Cu") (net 11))
 (via (at 118.65 79) (size 0.6) (drill 0.3) (layers "F.Cu" "B.Cu") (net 11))
 (via (at 119.552338 90.701039) (size 0.6) (drill 0.3) (layers "F.Cu" "B.Cu") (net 11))
 (segment (start 119.05 81.65) (end 118.85 81.85) (width 0.13) (layer "B.Cu") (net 11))
 (segment (start 118.85 81.85) (end 118.85 88.4) (width 0.13) (layer "B.Cu") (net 11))
 (segment (start 118.701039 90.701039) (end 119.552338 90.701039) (width 0.13) (layer "B.Cu") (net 11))
 (segment (start 117.9 89.9) (end 118.701039 90.701039) (width 0.13) (layer "B.Cu") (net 11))
 (segment (start 118.85 88.4) (end 117.9 89.35) (width 0.13) (layer "B.Cu") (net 11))
 (segment (start 119.05 79.4) (end 119.05 81.65) (width 0.13) (layer "B.Cu") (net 11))
 (segment (start 117.9 89.35) (end 117.9 89.9) (width 0.13) (layer "B.Cu") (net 11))
 (segment (start 118.65 79) (end 119.05 79.4) (width 0.13) (layer "B.Cu") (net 11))
 (segment (start 117.3 90.1) (end 116.400064 90.999936) (width 0.13) (layer "F.Cu") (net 4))
 (segment (start 116.400064 90.999936) (end 116.400064 91.974994) (width 0.13) (layer "F.Cu") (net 4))
 (segment (start 117.3 89.6) (end 117.3 90.1) (width 0.13) (layer "F.Cu") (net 4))
 (segment (start 118.45 81.35) (end 118.627821 81.35) (width 0.13) (layer "F.Cu") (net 4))
 (segment (start 118.627821 81.35) (end 119.634459 80.343362) (width 0.13) (layer "F.Cu") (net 4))
 (via (at 117.3 89.6) (size 0.6) (drill 0.3) (layers "F.Cu" "B.Cu") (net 4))
 (via (at 118.45 81.35) (size 0.6) (drill 0.3) (layers "F.Cu" "B.Cu") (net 4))
 (segment (start 117.3 89.6) (end 117.3 89.35) (width 0.13) (layer "B.Cu") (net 4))
 (segment (start 117.3 89.35) (end 118.45 88.2) (width 0.13) (layer "B.Cu") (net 4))
 (segment (start 118.45 88.2) (end 118.45 81.35) (width 0.13) (layer "B.Cu") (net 4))
 (segment (start 116.899936 91.050064) (end 116.899936 91.974994) (width 0.13) (layer "F.Cu") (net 3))
 (segment (start 115.7 88.65) (end 116 88.95) (width 0.13) (layer "F.Cu") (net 3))
 (segment (start 117.6 88.95) (end 117.9 89.25) (width 0.13) (layer "F.Cu") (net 3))
 (segment (start 117.9 89.25) (end 117.9 90.05) (width 0.13) (layer "F.Cu") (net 3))
 (segment (start 116.565541 87.456638) (end 115.7 88.322179) (width 0.13) (layer "F.Cu") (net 3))
 (segment (start 117.9 90.05) (end 116.899936 91.050064) (width 0.13) (layer "F.Cu") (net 3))
 (segment (start 116 88.95) (end 117.6 88.95) (width 0.13) (layer "F.Cu") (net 3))
 (segment (start 115.7 88.322179) (end 115.7 88.65) (width 0.13) (layer "F.Cu") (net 3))
 (segment (start 114.5 87.4) (end 114.600179 87.4) (width 0.13) (layer "F.Cu") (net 2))
 (segment (start 114.600179 87.4) (end 115.554541 86.445638) (width 0.13) (layer "F.Cu") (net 2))
 (segment (start 117.899936 93.35) (end 117.899936 91.974994) (width 0.13) (layer "F.Cu") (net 2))
 (via (at 117.899936 93.35) (size 0.6) (drill 0.3) (layers "F.Cu" "B.Cu") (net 2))
 (via (at 114.5 87.4) (size 0.6) (drill 0.3) (layers "F.Cu" "B.Cu") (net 2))
 (segment (start 117.899936 91.849936) (end 114.5 88.45) (width 0.13) (layer "B.Cu") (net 2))
 (segment (start 117.899936 93.35) (end 117.899936 91.849936) (width 0.13) (layer "B.Cu") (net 2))
 (segment (start 114.5 88.45) (end 114.5 87.4) (width 0.13) (layer "B.Cu") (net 2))
 (segment (start 118.400064 90.999936) (end 118.400064 91.974994) (width 0.13) (layer "F.Cu") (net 5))
 (segment (start 119.1 82.900179) (end 119.1 90.3) (width 0.13) (layer "F.Cu") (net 5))
 (segment (start 120.645638 81.354541) (end 119.1 82.900179) (width 0.13) (layer "F.Cu") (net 5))
 (segment (start 119.1 90.3) (end 118.400064 90.999936) (width 0.13) (layer "F.Cu") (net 5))
 (segment (start 113.6 86.377821) (end 114.543362 85.434459) (width 0.13) (layer "F.Cu") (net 1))
 (segment (start 113.6 87.4) (end 113.6 86.377821) (width 0.13) (layer "F.Cu") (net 1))
 (segment (start 115.899936 89.699936) (end 113.6 87.4) (width 0.13) (layer "F.Cu") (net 1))
 (segment (start 115.899936 91.974994) (end 115.899936 89.699936) (width 0.13) (layer "F.Cu") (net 1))
 (segment (start 120.65 83.25) (end 120.772179 83.25) (width 0.13) (layer "F.Cu") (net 6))
 (segment (start 117.400064 91.049936) (end 117.400064 91.974994) (width 0.13) (layer "F.Cu") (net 6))
 (segment (start 118.5 89.95) (end 117.400064 91.049936) (width 0.13) (layer "F.Cu") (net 6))
 (segment (start 118.5 89.6) (end 118.5 89.95) (width 0.13) (layer "F.Cu") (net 6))
 (segment (start 120.772179 83.25) (end 121.656638 82.365541) (width 0.13) (layer "F.Cu") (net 6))
 (via (at 118.5 89.6) (size 0.6) (drill 0.3) (layers "F.Cu" "B.Cu") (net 6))
 (via (at 120.65 83.25) (size 0.6) (drill 0.3) (layers "F.Cu" "B.Cu") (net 6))
 (segment (start 119.3 88.8) (end 119.3 84.6) (width 0.13) (layer "B.Cu") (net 6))
 (segment (start 119.3 84.6) (end 120.65 83.25) (width 0.13) (layer "B.Cu") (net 6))
 (segment (start 118.5 89.6) (end 119.3 88.8) (width 0.13) (layer "B.Cu") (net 6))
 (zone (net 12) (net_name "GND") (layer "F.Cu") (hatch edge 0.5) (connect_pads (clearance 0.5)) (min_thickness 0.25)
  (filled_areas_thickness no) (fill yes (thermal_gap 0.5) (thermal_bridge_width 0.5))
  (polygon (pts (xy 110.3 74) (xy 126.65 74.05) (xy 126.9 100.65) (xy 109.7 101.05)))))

